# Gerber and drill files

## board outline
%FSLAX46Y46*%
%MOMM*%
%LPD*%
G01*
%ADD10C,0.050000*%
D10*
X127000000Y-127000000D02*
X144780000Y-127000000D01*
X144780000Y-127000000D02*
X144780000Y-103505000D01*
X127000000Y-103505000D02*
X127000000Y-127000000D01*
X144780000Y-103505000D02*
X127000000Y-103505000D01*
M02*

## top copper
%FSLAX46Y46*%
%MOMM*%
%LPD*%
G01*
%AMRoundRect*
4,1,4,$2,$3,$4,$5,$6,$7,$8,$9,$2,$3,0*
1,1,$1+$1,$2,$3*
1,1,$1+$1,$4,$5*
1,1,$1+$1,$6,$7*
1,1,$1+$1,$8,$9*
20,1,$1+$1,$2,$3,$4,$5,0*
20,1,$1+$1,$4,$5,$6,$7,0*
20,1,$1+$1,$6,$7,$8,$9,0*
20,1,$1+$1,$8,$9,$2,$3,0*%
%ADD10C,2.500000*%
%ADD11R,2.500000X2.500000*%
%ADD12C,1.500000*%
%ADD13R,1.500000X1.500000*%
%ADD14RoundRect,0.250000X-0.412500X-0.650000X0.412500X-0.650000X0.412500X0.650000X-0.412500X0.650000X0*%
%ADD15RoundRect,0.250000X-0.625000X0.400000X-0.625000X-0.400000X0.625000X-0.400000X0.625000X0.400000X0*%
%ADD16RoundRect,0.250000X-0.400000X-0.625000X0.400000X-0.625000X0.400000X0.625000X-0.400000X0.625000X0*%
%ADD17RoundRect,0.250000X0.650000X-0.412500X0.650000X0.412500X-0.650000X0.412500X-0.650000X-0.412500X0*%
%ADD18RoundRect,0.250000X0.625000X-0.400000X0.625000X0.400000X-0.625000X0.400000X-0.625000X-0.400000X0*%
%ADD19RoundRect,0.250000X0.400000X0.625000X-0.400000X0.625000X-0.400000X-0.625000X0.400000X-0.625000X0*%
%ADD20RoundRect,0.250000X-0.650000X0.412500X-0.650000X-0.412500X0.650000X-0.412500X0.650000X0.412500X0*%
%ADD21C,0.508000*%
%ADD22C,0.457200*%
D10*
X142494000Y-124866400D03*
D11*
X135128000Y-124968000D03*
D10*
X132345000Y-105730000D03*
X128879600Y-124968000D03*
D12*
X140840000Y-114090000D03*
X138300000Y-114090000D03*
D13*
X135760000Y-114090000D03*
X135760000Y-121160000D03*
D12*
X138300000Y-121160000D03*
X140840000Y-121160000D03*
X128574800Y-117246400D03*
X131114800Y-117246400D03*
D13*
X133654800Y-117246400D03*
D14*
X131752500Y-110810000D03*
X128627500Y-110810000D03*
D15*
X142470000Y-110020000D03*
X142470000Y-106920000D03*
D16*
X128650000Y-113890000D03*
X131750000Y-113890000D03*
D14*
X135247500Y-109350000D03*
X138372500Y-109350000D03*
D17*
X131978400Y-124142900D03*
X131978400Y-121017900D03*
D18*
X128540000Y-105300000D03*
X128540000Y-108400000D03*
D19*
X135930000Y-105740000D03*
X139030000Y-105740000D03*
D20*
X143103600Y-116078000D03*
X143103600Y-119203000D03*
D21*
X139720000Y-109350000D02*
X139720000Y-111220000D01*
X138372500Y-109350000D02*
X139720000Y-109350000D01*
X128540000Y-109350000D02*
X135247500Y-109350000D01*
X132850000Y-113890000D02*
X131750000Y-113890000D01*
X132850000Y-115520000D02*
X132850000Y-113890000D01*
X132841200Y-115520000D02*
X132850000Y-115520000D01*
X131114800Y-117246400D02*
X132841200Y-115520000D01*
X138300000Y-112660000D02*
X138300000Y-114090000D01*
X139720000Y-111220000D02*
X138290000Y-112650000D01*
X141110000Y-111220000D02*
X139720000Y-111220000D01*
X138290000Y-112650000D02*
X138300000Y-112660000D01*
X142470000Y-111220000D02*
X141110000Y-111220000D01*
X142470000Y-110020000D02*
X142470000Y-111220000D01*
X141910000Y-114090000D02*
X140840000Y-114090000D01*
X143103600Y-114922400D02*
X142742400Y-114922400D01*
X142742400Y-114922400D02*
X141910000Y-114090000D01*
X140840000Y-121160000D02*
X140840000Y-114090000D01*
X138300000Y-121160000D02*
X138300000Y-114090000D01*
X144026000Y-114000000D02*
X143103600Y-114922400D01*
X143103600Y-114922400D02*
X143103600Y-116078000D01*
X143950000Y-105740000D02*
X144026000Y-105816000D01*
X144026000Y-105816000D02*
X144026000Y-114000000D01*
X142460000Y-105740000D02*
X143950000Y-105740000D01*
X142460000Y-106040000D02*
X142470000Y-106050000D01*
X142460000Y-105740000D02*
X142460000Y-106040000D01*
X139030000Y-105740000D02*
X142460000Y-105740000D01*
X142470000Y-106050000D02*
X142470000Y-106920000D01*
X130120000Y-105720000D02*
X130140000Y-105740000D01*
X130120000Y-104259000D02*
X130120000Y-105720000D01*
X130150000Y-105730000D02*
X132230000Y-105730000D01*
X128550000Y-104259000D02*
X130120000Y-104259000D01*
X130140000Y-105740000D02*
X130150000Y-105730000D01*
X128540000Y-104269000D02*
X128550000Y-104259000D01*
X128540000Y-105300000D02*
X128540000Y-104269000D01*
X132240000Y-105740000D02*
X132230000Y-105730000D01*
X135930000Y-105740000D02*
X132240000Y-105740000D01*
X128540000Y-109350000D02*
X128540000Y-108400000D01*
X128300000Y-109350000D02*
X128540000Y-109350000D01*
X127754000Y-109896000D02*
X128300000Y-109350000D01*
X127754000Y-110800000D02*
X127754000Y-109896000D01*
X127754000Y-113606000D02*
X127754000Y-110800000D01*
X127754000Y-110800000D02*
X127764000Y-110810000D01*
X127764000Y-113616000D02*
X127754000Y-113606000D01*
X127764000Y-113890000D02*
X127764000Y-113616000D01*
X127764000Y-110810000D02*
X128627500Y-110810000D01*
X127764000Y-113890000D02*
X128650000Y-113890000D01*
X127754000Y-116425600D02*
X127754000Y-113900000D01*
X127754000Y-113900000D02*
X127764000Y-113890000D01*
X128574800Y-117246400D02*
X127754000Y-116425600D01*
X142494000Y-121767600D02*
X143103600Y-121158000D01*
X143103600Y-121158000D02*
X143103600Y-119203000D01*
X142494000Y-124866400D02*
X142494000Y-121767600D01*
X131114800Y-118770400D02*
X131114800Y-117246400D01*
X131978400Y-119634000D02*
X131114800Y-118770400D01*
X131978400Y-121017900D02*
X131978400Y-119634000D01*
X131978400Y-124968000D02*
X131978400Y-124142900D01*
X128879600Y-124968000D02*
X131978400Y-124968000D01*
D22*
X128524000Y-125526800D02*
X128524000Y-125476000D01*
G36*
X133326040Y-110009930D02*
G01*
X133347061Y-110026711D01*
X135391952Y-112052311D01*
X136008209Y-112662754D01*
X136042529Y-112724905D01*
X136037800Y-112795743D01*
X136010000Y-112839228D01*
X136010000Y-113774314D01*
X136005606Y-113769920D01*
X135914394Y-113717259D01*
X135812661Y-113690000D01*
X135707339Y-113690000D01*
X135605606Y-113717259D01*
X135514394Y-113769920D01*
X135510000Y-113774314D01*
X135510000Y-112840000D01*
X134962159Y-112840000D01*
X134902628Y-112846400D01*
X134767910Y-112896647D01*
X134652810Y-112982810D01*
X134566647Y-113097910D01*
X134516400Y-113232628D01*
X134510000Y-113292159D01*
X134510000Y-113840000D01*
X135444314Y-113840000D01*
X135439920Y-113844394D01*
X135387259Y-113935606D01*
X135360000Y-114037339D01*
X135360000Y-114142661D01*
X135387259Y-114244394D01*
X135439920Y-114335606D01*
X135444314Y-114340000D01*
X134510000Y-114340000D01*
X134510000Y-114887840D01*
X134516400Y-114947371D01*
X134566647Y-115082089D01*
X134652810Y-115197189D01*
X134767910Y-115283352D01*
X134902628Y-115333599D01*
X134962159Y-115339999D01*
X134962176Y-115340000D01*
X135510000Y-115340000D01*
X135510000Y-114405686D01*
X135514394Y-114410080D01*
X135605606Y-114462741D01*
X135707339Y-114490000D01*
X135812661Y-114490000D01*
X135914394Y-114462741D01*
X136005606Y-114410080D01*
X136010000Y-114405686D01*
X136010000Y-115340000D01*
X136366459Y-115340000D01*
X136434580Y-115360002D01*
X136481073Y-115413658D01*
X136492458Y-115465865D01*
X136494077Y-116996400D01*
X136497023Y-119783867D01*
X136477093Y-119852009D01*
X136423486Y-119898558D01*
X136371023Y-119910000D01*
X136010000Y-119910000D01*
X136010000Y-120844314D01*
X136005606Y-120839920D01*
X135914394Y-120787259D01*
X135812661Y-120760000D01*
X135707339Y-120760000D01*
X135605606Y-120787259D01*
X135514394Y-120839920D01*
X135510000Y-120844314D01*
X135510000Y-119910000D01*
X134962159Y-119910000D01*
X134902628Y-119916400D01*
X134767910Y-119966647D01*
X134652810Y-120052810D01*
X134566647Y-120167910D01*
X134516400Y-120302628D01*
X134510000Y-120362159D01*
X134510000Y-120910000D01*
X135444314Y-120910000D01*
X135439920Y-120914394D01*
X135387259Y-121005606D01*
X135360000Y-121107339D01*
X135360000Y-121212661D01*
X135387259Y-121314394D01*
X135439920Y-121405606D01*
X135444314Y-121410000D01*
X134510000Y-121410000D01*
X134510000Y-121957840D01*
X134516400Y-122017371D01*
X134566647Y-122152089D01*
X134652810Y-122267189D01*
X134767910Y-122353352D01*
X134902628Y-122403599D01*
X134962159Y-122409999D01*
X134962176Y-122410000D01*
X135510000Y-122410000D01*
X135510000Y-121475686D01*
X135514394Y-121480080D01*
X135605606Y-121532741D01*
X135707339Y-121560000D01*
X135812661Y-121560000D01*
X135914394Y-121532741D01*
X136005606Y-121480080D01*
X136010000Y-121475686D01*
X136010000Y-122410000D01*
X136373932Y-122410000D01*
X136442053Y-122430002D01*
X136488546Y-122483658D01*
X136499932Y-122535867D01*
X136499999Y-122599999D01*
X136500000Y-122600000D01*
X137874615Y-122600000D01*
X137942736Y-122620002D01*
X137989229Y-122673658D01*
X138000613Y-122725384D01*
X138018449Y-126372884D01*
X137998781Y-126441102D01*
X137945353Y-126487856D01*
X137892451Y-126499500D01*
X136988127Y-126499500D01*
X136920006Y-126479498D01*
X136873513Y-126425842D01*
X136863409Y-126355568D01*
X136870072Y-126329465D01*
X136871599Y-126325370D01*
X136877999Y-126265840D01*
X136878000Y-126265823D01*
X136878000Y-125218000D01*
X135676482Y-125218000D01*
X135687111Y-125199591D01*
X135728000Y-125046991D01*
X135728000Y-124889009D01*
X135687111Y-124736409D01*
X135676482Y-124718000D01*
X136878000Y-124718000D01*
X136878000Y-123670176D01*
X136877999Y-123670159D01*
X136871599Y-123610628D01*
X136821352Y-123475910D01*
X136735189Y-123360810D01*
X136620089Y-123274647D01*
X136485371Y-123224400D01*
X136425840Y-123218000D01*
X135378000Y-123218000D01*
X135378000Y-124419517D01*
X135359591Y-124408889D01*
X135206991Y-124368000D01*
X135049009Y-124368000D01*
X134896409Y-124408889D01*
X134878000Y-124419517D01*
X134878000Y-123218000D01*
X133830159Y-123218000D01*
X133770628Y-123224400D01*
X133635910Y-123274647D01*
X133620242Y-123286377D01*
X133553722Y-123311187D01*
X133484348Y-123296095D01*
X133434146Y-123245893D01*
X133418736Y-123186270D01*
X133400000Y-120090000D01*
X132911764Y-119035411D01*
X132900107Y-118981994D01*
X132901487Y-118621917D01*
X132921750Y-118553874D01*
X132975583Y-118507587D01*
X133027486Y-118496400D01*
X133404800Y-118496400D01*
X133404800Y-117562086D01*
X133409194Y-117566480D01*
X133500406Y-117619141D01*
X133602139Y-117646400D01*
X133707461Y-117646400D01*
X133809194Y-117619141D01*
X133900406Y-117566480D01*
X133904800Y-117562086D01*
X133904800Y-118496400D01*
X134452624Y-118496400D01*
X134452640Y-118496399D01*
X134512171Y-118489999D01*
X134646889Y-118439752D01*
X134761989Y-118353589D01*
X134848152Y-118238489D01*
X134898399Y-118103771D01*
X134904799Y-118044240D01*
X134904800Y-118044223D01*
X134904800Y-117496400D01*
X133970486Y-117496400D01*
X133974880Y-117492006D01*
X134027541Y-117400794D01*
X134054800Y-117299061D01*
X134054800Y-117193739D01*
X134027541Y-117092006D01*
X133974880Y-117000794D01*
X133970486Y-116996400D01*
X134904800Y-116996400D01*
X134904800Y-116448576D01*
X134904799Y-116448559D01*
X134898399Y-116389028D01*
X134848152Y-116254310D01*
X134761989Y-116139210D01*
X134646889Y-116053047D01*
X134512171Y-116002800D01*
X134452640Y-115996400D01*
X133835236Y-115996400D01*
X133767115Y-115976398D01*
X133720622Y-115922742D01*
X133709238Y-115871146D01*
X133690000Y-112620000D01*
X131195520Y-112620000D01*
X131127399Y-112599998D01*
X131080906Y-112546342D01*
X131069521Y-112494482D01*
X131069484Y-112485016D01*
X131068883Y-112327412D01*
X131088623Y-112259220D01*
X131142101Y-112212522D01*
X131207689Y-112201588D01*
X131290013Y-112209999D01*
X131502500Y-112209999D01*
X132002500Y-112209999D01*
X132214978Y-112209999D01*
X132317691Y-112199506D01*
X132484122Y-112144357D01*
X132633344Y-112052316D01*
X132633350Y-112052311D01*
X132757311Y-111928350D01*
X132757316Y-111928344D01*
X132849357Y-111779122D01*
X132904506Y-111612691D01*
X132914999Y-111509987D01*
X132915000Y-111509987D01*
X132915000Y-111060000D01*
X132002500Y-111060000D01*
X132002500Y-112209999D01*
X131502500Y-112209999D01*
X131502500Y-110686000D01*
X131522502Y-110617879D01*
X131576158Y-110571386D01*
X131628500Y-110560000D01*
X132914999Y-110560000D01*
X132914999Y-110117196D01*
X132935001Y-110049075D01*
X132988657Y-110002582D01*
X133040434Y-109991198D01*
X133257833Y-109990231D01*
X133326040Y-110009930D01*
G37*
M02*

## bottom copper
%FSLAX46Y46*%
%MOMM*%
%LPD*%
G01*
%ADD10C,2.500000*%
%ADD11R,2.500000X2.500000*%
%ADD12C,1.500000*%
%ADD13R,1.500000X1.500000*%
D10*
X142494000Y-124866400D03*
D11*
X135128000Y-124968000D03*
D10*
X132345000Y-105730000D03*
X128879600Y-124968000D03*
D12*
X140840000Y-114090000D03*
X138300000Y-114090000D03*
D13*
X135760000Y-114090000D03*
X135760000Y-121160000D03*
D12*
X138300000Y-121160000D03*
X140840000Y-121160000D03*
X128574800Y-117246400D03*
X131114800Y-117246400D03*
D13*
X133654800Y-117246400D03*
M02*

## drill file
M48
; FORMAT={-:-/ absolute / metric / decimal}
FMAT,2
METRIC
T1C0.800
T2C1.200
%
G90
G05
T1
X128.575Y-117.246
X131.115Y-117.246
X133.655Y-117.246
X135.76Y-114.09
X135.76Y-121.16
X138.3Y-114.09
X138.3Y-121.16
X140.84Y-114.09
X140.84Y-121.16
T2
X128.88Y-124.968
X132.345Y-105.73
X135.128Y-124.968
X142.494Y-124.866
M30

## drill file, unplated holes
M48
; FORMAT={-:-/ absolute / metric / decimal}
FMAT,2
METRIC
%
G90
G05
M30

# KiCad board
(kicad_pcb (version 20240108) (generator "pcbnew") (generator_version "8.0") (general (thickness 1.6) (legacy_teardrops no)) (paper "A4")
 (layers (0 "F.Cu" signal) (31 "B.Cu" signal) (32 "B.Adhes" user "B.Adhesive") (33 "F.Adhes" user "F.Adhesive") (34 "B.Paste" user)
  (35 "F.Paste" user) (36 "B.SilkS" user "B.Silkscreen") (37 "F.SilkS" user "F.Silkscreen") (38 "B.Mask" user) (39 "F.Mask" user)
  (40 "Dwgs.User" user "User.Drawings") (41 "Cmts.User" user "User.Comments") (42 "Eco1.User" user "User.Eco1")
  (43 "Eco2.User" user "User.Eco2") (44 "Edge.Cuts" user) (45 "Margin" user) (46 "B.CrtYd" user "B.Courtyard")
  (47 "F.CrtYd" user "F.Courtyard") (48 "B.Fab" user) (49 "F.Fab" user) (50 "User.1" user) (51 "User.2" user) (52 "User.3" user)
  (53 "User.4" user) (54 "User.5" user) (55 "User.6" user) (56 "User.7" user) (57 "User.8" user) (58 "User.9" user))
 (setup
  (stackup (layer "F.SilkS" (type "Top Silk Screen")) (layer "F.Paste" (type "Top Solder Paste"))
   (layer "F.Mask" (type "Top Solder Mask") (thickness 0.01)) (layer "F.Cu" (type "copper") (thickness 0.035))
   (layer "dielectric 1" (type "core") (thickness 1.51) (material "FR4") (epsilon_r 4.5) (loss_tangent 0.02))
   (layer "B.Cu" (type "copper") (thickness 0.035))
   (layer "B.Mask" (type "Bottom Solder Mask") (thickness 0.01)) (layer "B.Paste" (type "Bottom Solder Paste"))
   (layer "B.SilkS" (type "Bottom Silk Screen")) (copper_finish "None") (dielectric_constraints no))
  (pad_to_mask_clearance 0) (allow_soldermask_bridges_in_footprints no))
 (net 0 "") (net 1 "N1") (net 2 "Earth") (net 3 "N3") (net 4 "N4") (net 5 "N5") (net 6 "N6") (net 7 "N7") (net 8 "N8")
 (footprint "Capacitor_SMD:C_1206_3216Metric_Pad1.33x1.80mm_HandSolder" (layer "F.Cu") (at 130.19 110.81)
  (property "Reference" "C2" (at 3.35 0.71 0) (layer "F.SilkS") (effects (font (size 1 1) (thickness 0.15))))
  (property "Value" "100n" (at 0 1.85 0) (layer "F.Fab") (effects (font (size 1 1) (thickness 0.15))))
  (pad "1" smd roundrect (at -1.5625 0) (size 1.325 1.8) (layers "F.Cu" "F.Paste" "F.Mask") (roundrect_rratio 0.188679) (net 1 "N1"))
  (pad "2" smd roundrect (at 1.5625 0) (size 1.325 1.8) (layers "F.Cu" "F.Paste" "F.Mask") (roundrect_rratio 0.188679) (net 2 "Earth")))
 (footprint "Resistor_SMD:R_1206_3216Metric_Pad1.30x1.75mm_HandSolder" (layer "F.Cu") (at 142.47 108.47 -90)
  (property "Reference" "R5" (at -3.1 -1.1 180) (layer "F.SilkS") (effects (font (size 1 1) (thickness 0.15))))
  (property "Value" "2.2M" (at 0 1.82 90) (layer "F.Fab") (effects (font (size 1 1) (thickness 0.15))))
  (pad "1" smd roundrect (at -1.55 0 270) (size 1.3 1.75) (layers "F.Cu" "F.Paste" "F.Mask") (roundrect_rratio 0.192308) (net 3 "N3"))
  (pad "2" smd roundrect (at 1.55 0 270) (size 1.3 1.75) (layers "F.Cu" "F.Paste" "F.Mask") (roundrect_rratio 0.192308) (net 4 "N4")))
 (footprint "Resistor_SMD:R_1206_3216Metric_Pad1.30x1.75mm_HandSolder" (layer "F.Cu") (at 130.2 113.89)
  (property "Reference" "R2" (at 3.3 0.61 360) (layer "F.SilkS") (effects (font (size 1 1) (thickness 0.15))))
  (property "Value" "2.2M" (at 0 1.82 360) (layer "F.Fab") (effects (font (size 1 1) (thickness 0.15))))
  (pad "1" smd roundrect (at -1.55 0) (size 1.3 1.75) (layers "F.Cu" "F.Paste" "F.Mask") (roundrect_rratio 0.192308) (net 1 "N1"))
  (pad "2" smd roundrect (at 1.55 0) (size 1.3 1.75) (layers "F.Cu" "F.Paste" "F.Mask") (roundrect_rratio 0.192308) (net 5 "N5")))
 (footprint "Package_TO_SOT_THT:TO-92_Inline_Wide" (layer "F.Cu") (at 133.6548 117.2464 180)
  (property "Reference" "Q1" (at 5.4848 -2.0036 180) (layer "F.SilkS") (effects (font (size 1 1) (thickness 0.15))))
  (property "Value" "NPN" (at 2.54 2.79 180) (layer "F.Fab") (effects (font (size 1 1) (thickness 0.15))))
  (pad "1" thru_hole rect (at 0 0 180) (size 1.5 1.5) (drill 0.8) (layers "*.Cu" "*.Mask") (remove_unused_layers no) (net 2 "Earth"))
  (pad "2" thru_hole circle (at 2.54 0 180) (size 1.5 1.5) (drill 0.8) (layers "*.Cu" "*.Mask") (remove_unused_layers no) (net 5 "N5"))
  (pad "3" thru_hole circle (at 5.08 0 180) (size 1.5 1.5) (drill 0.8) (layers "*.Cu" "*.Mask") (remove_unused_layers no) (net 1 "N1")))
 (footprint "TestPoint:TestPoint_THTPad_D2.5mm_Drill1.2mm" (layer "F.Cu") (at 132.345 105.73)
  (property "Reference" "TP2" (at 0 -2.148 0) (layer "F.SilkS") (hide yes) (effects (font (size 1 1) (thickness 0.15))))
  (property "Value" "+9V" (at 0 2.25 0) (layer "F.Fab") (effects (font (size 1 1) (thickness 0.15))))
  (pad "1" thru_hole circle (at 0 0) (size 2.5 2.5) (drill 1.2) (layers "*.Cu" "*.Mask") (remove_unused_layers no) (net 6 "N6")))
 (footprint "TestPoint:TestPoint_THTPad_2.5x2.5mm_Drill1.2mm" (layer "F.Cu") (at 135.128 124.968)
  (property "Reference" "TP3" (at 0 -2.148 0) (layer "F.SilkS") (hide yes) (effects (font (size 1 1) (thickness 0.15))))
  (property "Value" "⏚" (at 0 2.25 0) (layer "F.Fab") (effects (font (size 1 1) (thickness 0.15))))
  (pad "1" thru_hole rect (at 0 0) (size 2.5 2.5) (drill 1.2) (layers "*.Cu" "*.Mask") (remove_unused_layers no) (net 2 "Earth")))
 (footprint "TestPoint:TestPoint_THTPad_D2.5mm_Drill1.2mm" (layer "F.Cu") (at 142.494 124.8664)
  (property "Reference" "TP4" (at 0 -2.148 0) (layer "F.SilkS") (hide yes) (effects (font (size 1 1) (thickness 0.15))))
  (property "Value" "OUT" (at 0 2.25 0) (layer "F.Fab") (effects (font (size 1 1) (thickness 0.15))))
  (pad "1" thru_hole circle (at 0 0) (size 2.5 2.5) (drill 1.2) (layers "*.Cu" "*.Mask") (remove_unused_layers no) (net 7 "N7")))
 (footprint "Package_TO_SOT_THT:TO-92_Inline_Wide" (layer "F.Cu") (at 135.76 114.09)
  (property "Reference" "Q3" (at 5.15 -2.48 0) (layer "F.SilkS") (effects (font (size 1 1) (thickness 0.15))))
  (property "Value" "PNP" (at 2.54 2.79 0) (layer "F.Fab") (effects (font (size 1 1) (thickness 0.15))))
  (pad "1" thru_hole rect (at 0 0) (size 1.5 1.5) (drill 0.8) (layers "*.Cu" "*.Mask") (remove_unused_layers no) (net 2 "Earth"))
  (pad "2" thru_hole circle (at 2.54 0) (size 1.5 1.5) (drill 0.8) (layers "*.Cu" "*.Mask") (remove_unused_layers no) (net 4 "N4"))
  (pad "3" thru_hole circle (at 5.08 0) (size 1.5 1.5) (drill 0.8) (layers "*.Cu" "*.Mask") (remove_unused_layers no) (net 3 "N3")))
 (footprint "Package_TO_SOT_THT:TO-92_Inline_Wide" (layer "F.Cu") (at 135.76 121.16)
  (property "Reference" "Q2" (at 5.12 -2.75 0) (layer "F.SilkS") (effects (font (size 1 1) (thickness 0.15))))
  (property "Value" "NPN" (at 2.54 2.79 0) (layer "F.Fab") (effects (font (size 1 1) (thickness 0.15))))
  (pad "1" thru_hole rect (at 0 0) (size 1.5 1.5) (drill 0.8) (layers "*.Cu" "*.Mask") (remove_unused_layers no) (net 2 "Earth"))
  (pad "2" thru_hole circle (at 2.54 0) (size 1.5 1.5) (drill 0.8) (layers "*.Cu" "*.Mask") (remove_unused_layers no) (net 4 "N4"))
  (pad "3" thru_hole circle (at 5.08 0) (size 1.5 1.5) (drill 0.8) (layers "*.Cu" "*.Mask") (remove_unused_layers no) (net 3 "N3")))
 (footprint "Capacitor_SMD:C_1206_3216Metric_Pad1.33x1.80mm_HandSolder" (layer "F.Cu") (at 136.81 109.35)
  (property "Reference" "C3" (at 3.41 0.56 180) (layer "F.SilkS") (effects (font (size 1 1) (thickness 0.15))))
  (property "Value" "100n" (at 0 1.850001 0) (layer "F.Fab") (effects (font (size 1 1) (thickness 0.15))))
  (pad "1" smd roundrect (at -1.5625 0) (size 1.325 1.8) (layers "F.Cu" "F.Paste" "F.Mask") (roundrect_rratio 0.188679) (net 1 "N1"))
  (pad "2" smd roundrect (at 1.5625 0) (size 1.325 1.8) (layers "F.Cu" "F.Paste" "F.Mask") (roundrect_rratio 0.188679) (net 4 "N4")))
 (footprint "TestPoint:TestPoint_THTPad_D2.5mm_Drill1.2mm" (layer "F.Cu") (at 128.8796 124.968)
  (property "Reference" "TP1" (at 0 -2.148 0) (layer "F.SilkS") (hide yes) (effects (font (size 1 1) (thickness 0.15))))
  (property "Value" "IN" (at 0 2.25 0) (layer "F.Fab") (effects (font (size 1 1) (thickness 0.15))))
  (pad "1" thru_hole circle (at 0 0) (size 2.5 2.5) (drill 1.2) (layers "*.Cu" "*.Mask") (remove_unused_layers no) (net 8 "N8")))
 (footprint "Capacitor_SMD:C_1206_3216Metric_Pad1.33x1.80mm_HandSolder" (layer "F.Cu") (at 131.9784 122.5804 90)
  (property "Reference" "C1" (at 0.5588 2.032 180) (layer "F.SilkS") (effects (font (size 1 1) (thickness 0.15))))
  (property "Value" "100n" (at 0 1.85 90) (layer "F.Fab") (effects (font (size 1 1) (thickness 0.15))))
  (pad "1" smd roundrect (at -1.5625 0 90) (size 1.325 1.8) (layers "F.Cu" "F.Paste" "F.Mask") (roundrect_rratio 0.188679) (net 8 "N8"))
  (pad "2" smd roundrect (at 1.5625 0 90) (size 1.325 1.8) (layers "F.Cu" "F.Paste" "F.Mask") (roundrect_rratio 0.188679) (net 5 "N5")))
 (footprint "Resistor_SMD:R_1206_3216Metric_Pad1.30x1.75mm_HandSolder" (layer "F.Cu") (at 128.54 106.85 90)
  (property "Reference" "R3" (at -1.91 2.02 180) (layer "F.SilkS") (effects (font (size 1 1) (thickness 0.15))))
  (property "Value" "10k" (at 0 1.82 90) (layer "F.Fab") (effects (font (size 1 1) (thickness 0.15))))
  (pad "1" smd roundrect (at -1.55 0 90) (size 1.3 1.75) (layers "F.Cu" "F.Paste" "F.Mask") (roundrect_rratio 0.192308) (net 1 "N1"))
  (pad "2" smd roundrect (at 1.55 0 90) (size 1.3 1.75) (layers "F.Cu" "F.Paste" "F.Mask") (roundrect_rratio 0.192308) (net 6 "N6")))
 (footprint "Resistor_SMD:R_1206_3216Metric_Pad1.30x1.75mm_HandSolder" (layer "F.Cu") (at 137.48 105.74 180)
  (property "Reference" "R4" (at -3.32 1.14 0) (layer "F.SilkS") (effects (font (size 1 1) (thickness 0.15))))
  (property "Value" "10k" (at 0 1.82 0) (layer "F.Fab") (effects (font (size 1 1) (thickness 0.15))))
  (pad "1" smd roundrect (at -1.55 0 180) (size 1.3 1.75) (layers "F.Cu" "F.Paste" "F.Mask") (roundrect_rratio 0.192308) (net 3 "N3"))
  (pad "2" smd roundrect (at 1.55 0 180) (size 1.3 1.75) (layers "F.Cu" "F.Paste" "F.Mask") (roundrect_rratio 0.192308) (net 6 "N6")))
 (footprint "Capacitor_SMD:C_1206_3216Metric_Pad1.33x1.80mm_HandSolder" (layer "F.Cu") (at 143.1036 117.6405 -90)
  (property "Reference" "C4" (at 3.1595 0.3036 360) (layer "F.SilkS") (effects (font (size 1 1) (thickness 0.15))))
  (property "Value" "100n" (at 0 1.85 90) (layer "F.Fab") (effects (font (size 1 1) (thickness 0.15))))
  (pad "1" smd roundrect (at -1.5625 0 270) (size 1.325 1.8) (layers "F.Cu" "F.Paste" "F.Mask") (roundrect_rratio 0.188679) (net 3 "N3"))
  (pad "2" smd roundrect (at 1.5625 0 270) (size 1.325 1.8) (layers "F.Cu" "F.Paste" "F.Mask") (roundrect_rratio 0.188679) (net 7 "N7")))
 (gr_line (start 127 127) (end 144.78 127) (stroke (width 0.05) (type default)) (layer "Edge.Cuts"))
 (gr_line (start 144.78 127) (end 144.78 103.505) (stroke (width 0.05) (type default)) (layer "Edge.Cuts"))
 (gr_line (start 127 103.505) (end 127 127) (stroke (width 0.05) (type default)) (layer "Edge.Cuts"))
 (gr_line (start 144.78 103.505) (end 127 103.505) (stroke (width 0.05) (type default)) (layer "Edge.Cuts"))
 (segment (start 128.8796 124.968) (end 131.9784 124.968) (width 0.508) (layer "F.Cu") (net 8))
 (segment (start 128.524 125.5268) (end 128.524 125.476) (width 0.4572) (layer "F.Cu") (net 8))
 (segment (start 131.9784 124.968) (end 131.9784 124.1429) (width 0.508) (layer "F.Cu") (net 8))
 (segment (start 132.85 115.52) (end 132.85 113.89) (width 0.508) (layer "F.Cu") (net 5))
 (segment (start 132.85 113.89) (end 131.75 113.89) (width 0.508) (layer "F.Cu") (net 5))
 (segment (start 131.9784 121.0179) (end 131.9784 119.634) (width 0.508) (layer "F.Cu") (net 5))
 (segment (start 131.1148 117.2464) (end 132.8412 115.52) (width 0.508) (layer "F.Cu") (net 5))
 (segment (start 131.9784 119.634) (end 131.1148 118.7704) (width 0.508) (layer "F.Cu") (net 5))
 (segment (start 131.1148 118.7704) (end 131.1148 117.2464) (width 0.508) (layer "F.Cu") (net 5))
 (segment (start 132.8412 115.52) (end 132.85 115.52) (width 0.508) (layer "F.Cu") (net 5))
 (segment (start 127.754 110.8) (end 127.764 110.81) (width 0.508) (layer "F.Cu") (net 1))
 (segment (start 127.754 116.4256) (end 127.754 113.9) (width 0.508) (layer "F.Cu") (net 1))
 (segment (start 127.754 110.8) (end 127.754 109.896) (width 0.508) (layer "F.Cu") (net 1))
 (segment (start 127.764 113.89) (end 127.764 113.616) (width 0.508) (layer "F.Cu") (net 1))
 (segment (start 128.54 109.35) (end 135.2475 109.35) (width 0.508) (layer "F.Cu") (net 1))
 (segment (start 127.764 110.81) (end 128.6275 110.81) (width 0.508) (layer "F.Cu") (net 1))
 (segment (start 127.754 113.9) (end 127.764 113.89) (width 0.508) (layer "F.Cu") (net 1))
 (segment (start 128.3 109.35) (end 128.54 109.35) (width 0.508) (layer "F.Cu") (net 1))
 (segment (start 128.54 109.35) (end 128.54 108.4) (width 0.508) (layer "F.Cu") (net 1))
 (segment (start 127.754 113.606) (end 127.754 110.8) (width 0.508) (layer "F.Cu") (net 1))
 (segment (start 127.764 113.89) (end 128.65 113.89) (width 0.508) (layer "F.Cu") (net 1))
 (segment (start 127.764 113.616) (end 127.754 113.606) (width 0.508) (layer "F.Cu") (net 1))
 (segment (start 127.754 109.896) (end 128.3 109.35) (width 0.508) (layer "F.Cu") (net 1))
 (segment (start 128.5748 117.2464) (end 127.754 116.4256) (width 0.508) (layer "F.Cu") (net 1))
 (segment (start 138.3725 109.35) (end 139.72 109.35) (width 0.508) (layer "F.Cu") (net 4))
 (segment (start 142.47 110.02) (end 142.47 111.22) (width 0.508) (layer "F.Cu") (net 4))
 (segment (start 139.72 111.22) (end 138.29 112.65) (width 0.508) (layer "F.Cu") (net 4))
 (segment (start 141.11 111.22) (end 139.72 111.22) (width 0.508) (layer "F.Cu") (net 4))
 (segment (start 139.72 109.35) (end 139.72 111.22) (width 0.508) (layer "F.Cu") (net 4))
 (segment (start 142.47 111.22) (end 141.11 111.22) (width 0.508) (layer "F.Cu") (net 4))
 (segment (start 138.3 121.16) (end 138.3 114.09) (width 0.508) (layer "F.Cu") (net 4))
 (segment (start 138.29 112.65) (end 138.3 112.66) (width 0.508) (layer "F.Cu") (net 4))
 (segment (start 138.3 112.66) (end 138.3 114.09) (width 0.508) (layer "F.Cu") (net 4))
 (segment (start 142.46 105.74) (end 142.46 106.04) (width 0.508) (layer "F.Cu") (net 3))
 (segment (start 144.026 105.816) (end 144.026 114) (width 0.508) (layer "F.Cu") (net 3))
 (segment (start 142.7424 114.9224) (end 141.91 114.09) (width 0.508) (layer "F.Cu") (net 3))
 (segment (start 139.03 105.74) (end 142.46 105.74) (width 0.508) (layer "F.Cu") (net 3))
 (segment (start 143.95 105.74) (end 144.026 105.816) (width 0.508) (layer "F.Cu") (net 3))
 (segment (start 140.84 121.16) (end 140.84 114.09) (width 0.508) (layer "F.Cu") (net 3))
 (segment (start 142.46 106.04) (end 142.47 106.05) (width 0.508) (layer "F.Cu") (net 3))
 (segment (start 142.47 106.05) (end 142.47 106.92) (width 0.508) (layer "F.Cu") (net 3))
 (segment (start 141.91 114.09) (end 140.84 114.09) (width 0.508) (layer "F.Cu") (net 3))
 (segment (start 142.46 105.74) (end 143.95 105.74) (width 0.508) (layer "F.Cu") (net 3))
 (segment (start 143.1036 114.9224) (end 143.1036 116.078) (width 0.508) (layer "F.Cu") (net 3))
 (segment (start 144.026 114) (end 143.1036 114.9224) (width 0.508) (layer "F.Cu") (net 3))
 (segment (start 143.1036 114.9224) (end 142.7424 114.9224) (width 0.508) (layer "F.Cu") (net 3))
 (segment (start 143.1036 121.158) (end 143.1036 119.203) (width 0.508) (layer "F.Cu") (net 7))
 (segment (start 142.494 121.7676) (end 143.1036 121.158) (width 0.508) (layer "F.Cu") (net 7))
 (segment (start 142.494 124.8664) (end 142.494 121.7676) (width 0.508) (layer "F.Cu") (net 7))
 (segment (start 128.55 104.259) (end 130.12 104.259) (width 0.508) (layer "F.Cu") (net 6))
 (segment (start 130.12 104.259) (end 130.12 105.72) (width 0.508) (layer "F.Cu") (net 6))
 (segment (start 130.12 105.72) (end 130.14 105.74) (width 0.508) (layer "F.Cu") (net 6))
 (segment (start 130.14 105.74) (end 130.15 105.73) (width 0.508) (layer "F.Cu") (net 6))
 (segment (start 135.93 105.74) (end 132.24 105.74) (width 0.508) (layer "F.Cu") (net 6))
 (segment (start 128.54 105.3) (end 128.54 104.269) (width 0.508) (layer "F.Cu") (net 6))
 (segment (start 130.15 105.73) (end 132.23 105.73) (width 0.508) (layer "F.Cu") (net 6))
 (segment (start 128.54 104.269) (end 128.55 104.259) (width 0.508) (layer "F.Cu") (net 6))
 (segment (start 132.24 105.74) (end 132.23 105.73) (width 0.508) (layer "F.Cu") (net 6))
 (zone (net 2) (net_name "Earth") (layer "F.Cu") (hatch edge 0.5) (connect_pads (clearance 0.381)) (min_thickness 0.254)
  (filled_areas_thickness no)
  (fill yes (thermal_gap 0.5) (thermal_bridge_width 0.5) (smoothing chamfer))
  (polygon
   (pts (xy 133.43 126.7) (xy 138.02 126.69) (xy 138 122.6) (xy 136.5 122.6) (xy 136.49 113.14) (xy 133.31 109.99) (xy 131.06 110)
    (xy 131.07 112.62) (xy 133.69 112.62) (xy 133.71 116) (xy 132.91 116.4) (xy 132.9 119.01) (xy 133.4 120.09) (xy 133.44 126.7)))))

